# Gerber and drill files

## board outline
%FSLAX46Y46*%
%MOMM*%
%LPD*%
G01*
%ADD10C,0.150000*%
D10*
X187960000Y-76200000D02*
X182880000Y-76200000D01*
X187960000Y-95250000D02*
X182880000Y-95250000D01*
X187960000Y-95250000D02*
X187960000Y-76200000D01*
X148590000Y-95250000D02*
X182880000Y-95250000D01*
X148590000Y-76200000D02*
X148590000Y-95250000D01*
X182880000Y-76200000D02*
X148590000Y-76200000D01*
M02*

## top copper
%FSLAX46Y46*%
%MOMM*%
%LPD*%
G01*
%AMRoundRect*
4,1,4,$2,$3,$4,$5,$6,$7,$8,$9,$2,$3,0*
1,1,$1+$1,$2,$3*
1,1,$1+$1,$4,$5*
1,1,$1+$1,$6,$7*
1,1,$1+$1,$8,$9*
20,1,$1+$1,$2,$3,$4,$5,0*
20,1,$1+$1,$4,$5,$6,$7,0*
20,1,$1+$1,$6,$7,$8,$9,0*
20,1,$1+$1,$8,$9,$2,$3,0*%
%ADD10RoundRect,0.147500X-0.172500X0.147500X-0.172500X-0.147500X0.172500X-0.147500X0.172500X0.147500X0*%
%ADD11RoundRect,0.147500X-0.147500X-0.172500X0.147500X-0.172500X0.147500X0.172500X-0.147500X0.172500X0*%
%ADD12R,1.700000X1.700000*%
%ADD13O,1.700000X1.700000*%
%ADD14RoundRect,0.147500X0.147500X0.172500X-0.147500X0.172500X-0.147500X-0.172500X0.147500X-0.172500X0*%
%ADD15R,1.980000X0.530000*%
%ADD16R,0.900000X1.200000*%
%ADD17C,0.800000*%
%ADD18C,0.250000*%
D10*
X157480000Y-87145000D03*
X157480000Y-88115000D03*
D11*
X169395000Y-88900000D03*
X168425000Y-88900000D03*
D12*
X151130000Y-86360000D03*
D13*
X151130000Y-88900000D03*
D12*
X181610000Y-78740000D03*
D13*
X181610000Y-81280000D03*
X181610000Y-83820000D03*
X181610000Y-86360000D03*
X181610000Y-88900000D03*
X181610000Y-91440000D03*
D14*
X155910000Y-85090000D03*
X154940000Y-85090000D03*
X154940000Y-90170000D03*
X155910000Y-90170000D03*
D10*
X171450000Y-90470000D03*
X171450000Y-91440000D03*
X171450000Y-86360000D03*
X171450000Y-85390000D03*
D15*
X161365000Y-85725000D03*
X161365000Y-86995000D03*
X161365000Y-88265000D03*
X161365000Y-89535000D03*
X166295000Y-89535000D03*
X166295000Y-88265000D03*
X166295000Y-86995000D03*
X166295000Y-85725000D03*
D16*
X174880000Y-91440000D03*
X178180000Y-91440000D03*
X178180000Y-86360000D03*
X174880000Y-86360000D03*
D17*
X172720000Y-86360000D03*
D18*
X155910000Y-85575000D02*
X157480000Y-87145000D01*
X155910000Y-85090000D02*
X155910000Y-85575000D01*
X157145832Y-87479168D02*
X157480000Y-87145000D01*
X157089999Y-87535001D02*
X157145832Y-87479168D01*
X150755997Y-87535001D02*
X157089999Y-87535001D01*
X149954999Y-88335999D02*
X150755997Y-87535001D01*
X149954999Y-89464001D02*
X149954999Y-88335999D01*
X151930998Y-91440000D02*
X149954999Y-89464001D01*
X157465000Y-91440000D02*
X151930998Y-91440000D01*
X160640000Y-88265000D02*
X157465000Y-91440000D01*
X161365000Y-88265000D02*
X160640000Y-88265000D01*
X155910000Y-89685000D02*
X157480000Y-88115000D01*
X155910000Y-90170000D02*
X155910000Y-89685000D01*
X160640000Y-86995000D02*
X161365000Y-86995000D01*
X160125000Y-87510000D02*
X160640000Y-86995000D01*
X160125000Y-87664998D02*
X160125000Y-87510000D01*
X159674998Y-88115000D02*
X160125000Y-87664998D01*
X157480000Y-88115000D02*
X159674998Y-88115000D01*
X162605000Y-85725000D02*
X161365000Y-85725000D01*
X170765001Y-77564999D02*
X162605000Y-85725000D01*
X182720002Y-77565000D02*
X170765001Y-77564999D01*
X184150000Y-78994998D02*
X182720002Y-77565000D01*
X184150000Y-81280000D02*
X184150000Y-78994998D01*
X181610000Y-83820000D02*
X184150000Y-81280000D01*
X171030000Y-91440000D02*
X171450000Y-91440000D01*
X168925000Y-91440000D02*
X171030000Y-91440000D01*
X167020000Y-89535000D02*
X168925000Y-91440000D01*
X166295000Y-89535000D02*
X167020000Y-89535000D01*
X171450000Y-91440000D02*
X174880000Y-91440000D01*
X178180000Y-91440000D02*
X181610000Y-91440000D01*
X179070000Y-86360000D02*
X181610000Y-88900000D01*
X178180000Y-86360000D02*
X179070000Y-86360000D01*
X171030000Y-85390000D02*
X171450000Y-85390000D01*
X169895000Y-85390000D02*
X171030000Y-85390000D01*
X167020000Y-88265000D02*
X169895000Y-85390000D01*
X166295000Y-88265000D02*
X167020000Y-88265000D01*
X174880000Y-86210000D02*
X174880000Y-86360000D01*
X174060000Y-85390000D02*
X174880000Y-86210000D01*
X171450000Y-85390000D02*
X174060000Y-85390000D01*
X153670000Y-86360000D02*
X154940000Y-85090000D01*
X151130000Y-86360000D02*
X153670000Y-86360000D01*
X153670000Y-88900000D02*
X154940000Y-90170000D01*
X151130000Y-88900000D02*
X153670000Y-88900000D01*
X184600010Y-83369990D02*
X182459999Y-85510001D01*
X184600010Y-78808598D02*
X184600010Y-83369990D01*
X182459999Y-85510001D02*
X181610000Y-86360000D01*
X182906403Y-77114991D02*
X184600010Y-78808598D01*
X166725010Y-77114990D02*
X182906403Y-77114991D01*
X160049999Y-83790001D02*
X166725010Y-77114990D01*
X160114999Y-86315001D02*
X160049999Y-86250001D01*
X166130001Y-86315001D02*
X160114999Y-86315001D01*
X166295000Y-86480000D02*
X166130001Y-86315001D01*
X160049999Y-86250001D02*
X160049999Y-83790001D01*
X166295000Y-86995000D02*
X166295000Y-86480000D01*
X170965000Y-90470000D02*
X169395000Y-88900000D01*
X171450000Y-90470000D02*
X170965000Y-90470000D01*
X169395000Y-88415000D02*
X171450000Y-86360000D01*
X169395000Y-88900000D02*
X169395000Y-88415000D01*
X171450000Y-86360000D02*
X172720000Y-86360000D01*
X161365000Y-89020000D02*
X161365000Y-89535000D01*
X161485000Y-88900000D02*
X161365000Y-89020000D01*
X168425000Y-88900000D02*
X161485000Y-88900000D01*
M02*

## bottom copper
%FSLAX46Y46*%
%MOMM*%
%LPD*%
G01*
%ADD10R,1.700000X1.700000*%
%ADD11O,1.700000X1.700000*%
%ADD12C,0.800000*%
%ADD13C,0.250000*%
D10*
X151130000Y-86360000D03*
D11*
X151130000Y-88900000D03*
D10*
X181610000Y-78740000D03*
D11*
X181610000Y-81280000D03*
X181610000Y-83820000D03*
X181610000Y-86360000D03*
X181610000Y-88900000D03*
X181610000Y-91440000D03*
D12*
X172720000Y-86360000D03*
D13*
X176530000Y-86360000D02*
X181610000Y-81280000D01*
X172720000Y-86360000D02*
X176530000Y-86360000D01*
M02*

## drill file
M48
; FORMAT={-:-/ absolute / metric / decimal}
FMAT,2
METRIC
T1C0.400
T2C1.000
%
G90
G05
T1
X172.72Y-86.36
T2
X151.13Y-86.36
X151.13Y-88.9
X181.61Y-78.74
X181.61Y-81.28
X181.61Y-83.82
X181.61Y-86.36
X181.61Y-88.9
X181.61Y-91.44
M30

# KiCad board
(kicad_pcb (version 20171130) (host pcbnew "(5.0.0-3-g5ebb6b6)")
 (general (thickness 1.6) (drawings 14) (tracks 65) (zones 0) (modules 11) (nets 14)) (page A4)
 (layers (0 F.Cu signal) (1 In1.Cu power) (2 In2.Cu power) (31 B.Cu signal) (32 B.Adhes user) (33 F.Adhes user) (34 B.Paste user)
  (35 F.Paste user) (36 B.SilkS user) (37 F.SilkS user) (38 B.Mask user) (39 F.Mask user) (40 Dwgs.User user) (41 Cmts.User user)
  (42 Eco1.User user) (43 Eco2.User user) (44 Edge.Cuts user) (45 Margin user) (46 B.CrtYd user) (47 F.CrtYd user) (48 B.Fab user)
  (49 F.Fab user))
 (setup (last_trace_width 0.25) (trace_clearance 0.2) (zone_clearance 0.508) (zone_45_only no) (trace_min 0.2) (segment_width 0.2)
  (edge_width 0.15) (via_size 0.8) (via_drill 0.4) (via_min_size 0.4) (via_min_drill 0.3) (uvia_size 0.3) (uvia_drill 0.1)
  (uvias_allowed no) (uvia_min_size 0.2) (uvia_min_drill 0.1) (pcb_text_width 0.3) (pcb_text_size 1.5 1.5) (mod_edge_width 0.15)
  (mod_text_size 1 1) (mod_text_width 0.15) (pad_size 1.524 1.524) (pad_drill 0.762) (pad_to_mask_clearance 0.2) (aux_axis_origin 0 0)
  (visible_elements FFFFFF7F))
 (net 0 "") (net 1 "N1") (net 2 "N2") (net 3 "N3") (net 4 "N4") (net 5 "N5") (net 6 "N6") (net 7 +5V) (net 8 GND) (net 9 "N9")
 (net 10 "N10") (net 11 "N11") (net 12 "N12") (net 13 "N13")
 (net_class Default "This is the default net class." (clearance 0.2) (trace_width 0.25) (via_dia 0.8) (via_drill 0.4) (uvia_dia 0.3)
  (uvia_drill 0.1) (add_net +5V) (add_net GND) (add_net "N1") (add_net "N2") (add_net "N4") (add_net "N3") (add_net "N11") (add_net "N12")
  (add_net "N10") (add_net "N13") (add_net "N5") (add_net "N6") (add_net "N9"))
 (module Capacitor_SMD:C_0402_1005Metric (layer F.Cu) (at 157.48 87.63 270)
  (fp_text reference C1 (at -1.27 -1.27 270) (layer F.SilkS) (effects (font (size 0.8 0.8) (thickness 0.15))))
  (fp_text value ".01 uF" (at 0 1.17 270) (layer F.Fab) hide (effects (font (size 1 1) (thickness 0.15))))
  (pad 1 smd roundrect (at -0.485 0 270) (size 0.59 0.64) (layers F.Cu F.Paste F.Mask) (roundrect_rratio 0.25) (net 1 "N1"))
  (pad 2 smd roundrect (at 0.485 0 270) (size 0.59 0.64) (layers F.Cu F.Paste F.Mask) (roundrect_rratio 0.25) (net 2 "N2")))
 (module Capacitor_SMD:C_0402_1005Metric (layer F.Cu) (at 168.91 88.9)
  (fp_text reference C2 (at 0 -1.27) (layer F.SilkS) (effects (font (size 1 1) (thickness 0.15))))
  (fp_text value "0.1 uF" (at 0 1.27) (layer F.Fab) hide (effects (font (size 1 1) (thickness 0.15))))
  (pad 2 smd roundrect (at 0.485 0) (size 0.59 0.64) (layers F.Cu F.Paste F.Mask) (roundrect_rratio 0.25) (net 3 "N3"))
  (pad 1 smd roundrect (at -0.485 0) (size 0.59 0.64) (layers F.Cu F.Paste F.Mask) (roundrect_rratio 0.25) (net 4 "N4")))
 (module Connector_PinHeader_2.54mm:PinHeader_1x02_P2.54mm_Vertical (layer F.Cu) (at 151.13 86.36)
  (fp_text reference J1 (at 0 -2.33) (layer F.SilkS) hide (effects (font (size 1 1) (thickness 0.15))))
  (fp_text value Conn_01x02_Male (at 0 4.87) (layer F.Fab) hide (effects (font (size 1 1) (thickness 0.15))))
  (pad 1 thru_hole rect (at 0 0) (size 1.7 1.7) (drill 1) (layers *.Cu *.Mask) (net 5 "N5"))
  (pad 2 thru_hole oval (at 0 2.54) (size 1.7 1.7) (drill 1) (layers *.Cu *.Mask) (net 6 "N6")))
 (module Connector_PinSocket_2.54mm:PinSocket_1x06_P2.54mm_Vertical (layer F.Cu) (at 181.61 78.74)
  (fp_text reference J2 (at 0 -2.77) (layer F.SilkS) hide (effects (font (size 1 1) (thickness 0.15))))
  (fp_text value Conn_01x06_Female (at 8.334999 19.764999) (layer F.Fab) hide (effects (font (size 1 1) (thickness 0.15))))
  (pad 1 thru_hole rect (at 0 0) (size 1.7 1.7) (drill 1) (layers *.Cu *.Mask) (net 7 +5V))
  (pad 2 thru_hole oval (at 0 2.54) (size 1.7 1.7) (drill 1) (layers *.Cu *.Mask) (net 3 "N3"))
  (pad 3 thru_hole oval (at 0 5.08) (size 1.7 1.7) (drill 1) (layers *.Cu *.Mask) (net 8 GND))
  (pad 4 thru_hole oval (at 0 7.62) (size 1.7 1.7) (drill 1) (layers *.Cu *.Mask) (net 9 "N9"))
  (pad 5 thru_hole oval (at 0 10.16) (size 1.7 1.7) (drill 1) (layers *.Cu *.Mask) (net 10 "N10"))
  (pad 6 thru_hole oval (at 0 12.7) (size 1.7 1.7) (drill 1) (layers *.Cu *.Mask) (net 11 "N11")))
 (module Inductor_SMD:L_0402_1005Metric (layer F.Cu) (at 155.425 85.09 180)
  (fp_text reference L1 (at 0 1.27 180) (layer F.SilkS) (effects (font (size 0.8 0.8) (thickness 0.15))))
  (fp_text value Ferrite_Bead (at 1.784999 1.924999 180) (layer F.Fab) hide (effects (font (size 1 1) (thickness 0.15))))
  (pad 1 smd roundrect (at -0.485 0 180) (size 0.59 0.64) (layers F.Cu F.Paste F.Mask) (roundrect_rratio 0.25) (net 1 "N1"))
  (pad 2 smd roundrect (at 0.485 0 180) (size 0.59 0.64) (layers F.Cu F.Paste F.Mask) (roundrect_rratio 0.25) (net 5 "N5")))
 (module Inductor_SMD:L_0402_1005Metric (layer F.Cu) (at 155.425 90.17 180)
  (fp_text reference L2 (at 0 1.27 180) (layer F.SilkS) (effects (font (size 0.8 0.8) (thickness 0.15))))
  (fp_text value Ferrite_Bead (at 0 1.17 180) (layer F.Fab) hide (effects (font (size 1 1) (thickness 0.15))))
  (pad 2 smd roundrect (at 0.485 0 180) (size 0.59 0.64) (layers F.Cu F.Paste F.Mask) (roundrect_rratio 0.25) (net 6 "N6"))
  (pad 1 smd roundrect (at -0.485 0 180) (size 0.59 0.64) (layers F.Cu F.Paste F.Mask) (roundrect_rratio 0.25) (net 2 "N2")))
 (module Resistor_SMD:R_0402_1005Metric (layer F.Cu) (at 171.45 90.955 270)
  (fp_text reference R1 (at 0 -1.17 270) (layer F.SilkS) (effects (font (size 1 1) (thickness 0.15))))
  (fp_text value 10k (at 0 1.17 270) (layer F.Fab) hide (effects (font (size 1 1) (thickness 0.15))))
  (pad 1 smd roundrect (at -0.485 0 270) (size 0.59 0.64) (layers F.Cu F.Paste F.Mask) (roundrect_rratio 0.25) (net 3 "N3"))
  (pad 2 smd roundrect (at 0.485 0 270) (size 0.59 0.64) (layers F.Cu F.Paste F.Mask) (roundrect_rratio 0.25) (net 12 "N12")))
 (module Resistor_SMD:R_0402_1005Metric (layer F.Cu) (at 171.45 85.875 270)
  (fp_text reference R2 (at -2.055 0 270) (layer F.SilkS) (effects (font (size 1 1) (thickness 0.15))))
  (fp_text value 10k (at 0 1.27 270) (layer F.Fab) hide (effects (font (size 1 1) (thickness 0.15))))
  (pad 2 smd roundrect (at 0.485 0 270) (size 0.59 0.64) (layers F.Cu F.Paste F.Mask) (roundrect_rratio 0.25) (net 3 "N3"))
  (pad 1 smd roundrect (at -0.485 0 270) (size 0.59 0.64) (layers F.Cu F.Paste F.Mask) (roundrect_rratio 0.25) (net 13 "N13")))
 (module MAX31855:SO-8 (layer F.Cu) (at 163.83 87.63)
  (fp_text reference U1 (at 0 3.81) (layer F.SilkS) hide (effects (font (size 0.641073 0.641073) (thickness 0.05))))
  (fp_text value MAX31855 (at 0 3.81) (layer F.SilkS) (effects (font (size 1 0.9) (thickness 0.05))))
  (pad 1 smd rect (at -2.465 -1.905) (size 1.98 0.53) (layers F.Cu F.Paste F.Mask) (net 8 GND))
  (pad 2 smd rect (at -2.465 -0.635) (size 1.98 0.53) (layers F.Cu F.Paste F.Mask) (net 2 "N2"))
  (pad 3 smd rect (at -2.465 0.635) (size 1.98 0.53) (layers F.Cu F.Paste F.Mask) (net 1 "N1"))
  (pad 4 smd rect (at -2.465 1.905) (size 1.98 0.53) (layers F.Cu F.Paste F.Mask) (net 4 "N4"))
  (pad 5 smd rect (at 2.465 1.905) (size 1.98 0.53) (layers F.Cu F.Paste F.Mask) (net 12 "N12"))
  (pad 6 smd rect (at 2.465 0.635) (size 1.98 0.53) (layers F.Cu F.Paste F.Mask) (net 13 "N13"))
  (pad 7 smd rect (at 2.465 -0.635) (size 1.98 0.53) (layers F.Cu F.Paste F.Mask) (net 9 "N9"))
  (pad 8 smd rect (at 2.465 -1.905) (size 1.98 0.53) (layers F.Cu F.Paste F.Mask)))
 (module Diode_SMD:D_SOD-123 (layer F.Cu) (at 176.53 91.44 180)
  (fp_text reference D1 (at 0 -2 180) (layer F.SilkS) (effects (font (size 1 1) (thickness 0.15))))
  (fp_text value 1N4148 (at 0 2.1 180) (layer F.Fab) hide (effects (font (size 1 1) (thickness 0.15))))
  (pad 2 smd rect (at 1.65 0 180) (size 0.9 1.2) (layers F.Cu F.Paste F.Mask) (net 12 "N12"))
  (pad 1 smd rect (at -1.65 0 180) (size 0.9 1.2) (layers F.Cu F.Paste F.Mask) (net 11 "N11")))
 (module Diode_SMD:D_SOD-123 (layer F.Cu) (at 176.53 86.36 180)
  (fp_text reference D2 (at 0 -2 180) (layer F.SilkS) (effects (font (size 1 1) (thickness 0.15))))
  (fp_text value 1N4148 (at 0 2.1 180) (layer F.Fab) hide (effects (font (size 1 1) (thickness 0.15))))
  (pad 1 smd rect (at -1.65 0 180) (size 0.9 1.2) (layers F.Cu F.Paste F.Mask) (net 10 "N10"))
  (pad 2 smd rect (at 1.65 0 180) (size 0.9 1.2) (layers F.Cu F.Paste F.Mask) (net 13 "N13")))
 (gr_line (start 187.96 76.2) (end 182.88 76.2) (layer Edge.Cuts) (width 0.15))
 (gr_line (start 187.96 95.25) (end 182.88 95.25) (layer Edge.Cuts) (width 0.15))
 (gr_line (start 187.96 95.25) (end 187.96 76.2) (layer Edge.Cuts) (width 0.15))
 (gr_line (start 148.59 95.25) (end 182.88 95.25) (layer Edge.Cuts) (width 0.15))
 (gr_line (start 148.59 76.2) (end 148.59 95.25) (layer Edge.Cuts) (width 0.15))
 (gr_line (start 182.88 76.2) (end 148.59 76.2) (layer Edge.Cuts) (width 0.15))
 (segment (start 155.91 85.575) (end 157.48 87.145) (width 0.25) (layer F.Cu) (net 1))
 (segment (start 155.91 85.09) (end 155.91 85.575) (width 0.25) (layer F.Cu) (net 1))
 (segment (start 157.145832 87.479168) (end 157.48 87.145) (width 0.25) (layer F.Cu) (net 1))
 (segment (start 157.089999 87.535001) (end 157.145832 87.479168) (width 0.25) (layer F.Cu) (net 1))
 (segment (start 150.755997 87.535001) (end 157.089999 87.535001) (width 0.25) (layer F.Cu) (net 1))
 (segment (start 149.954999 88.335999) (end 150.755997 87.535001) (width 0.25) (layer F.Cu) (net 1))
 (segment (start 149.954999 89.464001) (end 149.954999 88.335999) (width 0.25) (layer F.Cu) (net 1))
 (segment (start 151.930998 91.44) (end 149.954999 89.464001) (width 0.25) (layer F.Cu) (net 1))
 (segment (start 157.465 91.44) (end 151.930998 91.44) (width 0.25) (layer F.Cu) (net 1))
 (segment (start 160.64 88.265) (end 157.465 91.44) (width 0.25) (layer F.Cu) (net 1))
 (segment (start 161.365 88.265) (end 160.64 88.265) (width 0.25) (layer F.Cu) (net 1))
 (segment (start 155.91 89.685) (end 157.48 88.115) (width 0.25) (layer F.Cu) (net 2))
 (segment (start 155.91 90.17) (end 155.91 89.685) (width 0.25) (layer F.Cu) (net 2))
 (segment (start 160.64 86.995) (end 161.365 86.995) (width 0.25) (layer F.Cu) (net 2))
 (segment (start 160.125 87.51) (end 160.64 86.995) (width 0.25) (layer F.Cu) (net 2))
 (segment (start 160.125 87.664998) (end 160.125 87.51) (width 0.25) (layer F.Cu) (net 2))
 (segment (start 159.674998 88.115) (end 160.125 87.664998) (width 0.25) (layer F.Cu) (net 2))
 (segment (start 157.48 88.115) (end 159.674998 88.115) (width 0.25) (layer F.Cu) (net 2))
 (segment (start 162.605 85.725) (end 161.365 85.725) (width 0.25) (layer F.Cu) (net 8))
 (segment (start 170.765001 77.564999) (end 162.605 85.725) (width 0.25) (layer F.Cu) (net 8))
 (segment (start 182.720002 77.565) (end 170.765001 77.564999) (width 0.25) (layer F.Cu) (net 8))
 (segment (start 184.15 78.994998) (end 182.720002 77.565) (width 0.25) (layer F.Cu) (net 8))
 (segment (start 184.15 81.28) (end 184.15 78.994998) (width 0.25) (layer F.Cu) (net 8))
 (segment (start 181.61 83.82) (end 184.15 81.28) (width 0.25) (layer F.Cu) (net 8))
 (segment (start 171.03 91.44) (end 171.45 91.44) (width 0.25) (layer F.Cu) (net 12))
 (segment (start 168.925 91.44) (end 171.03 91.44) (width 0.25) (layer F.Cu) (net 12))
 (segment (start 167.02 89.535) (end 168.925 91.44) (width 0.25) (layer F.Cu) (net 12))
 (segment (start 166.295 89.535) (end 167.02 89.535) (width 0.25) (layer F.Cu) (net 12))
 (segment (start 171.45 91.44) (end 174.88 91.44) (width 0.25) (layer F.Cu) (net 12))
 (segment (start 178.18 91.44) (end 181.61 91.44) (width 0.25) (layer F.Cu) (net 11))
 (segment (start 179.07 86.36) (end 181.61 88.9) (width 0.25) (layer F.Cu) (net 10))
 (segment (start 178.18 86.36) (end 179.07 86.36) (width 0.25) (layer F.Cu) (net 10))
 (segment (start 171.03 85.39) (end 171.45 85.39) (width 0.25) (layer F.Cu) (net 13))
 (segment (start 169.895 85.39) (end 171.03 85.39) (width 0.25) (layer F.Cu) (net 13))
 (segment (start 167.02 88.265) (end 169.895 85.39) (width 0.25) (layer F.Cu) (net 13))
 (segment (start 166.295 88.265) (end 167.02 88.265) (width 0.25) (layer F.Cu) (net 13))
 (segment (start 174.88 86.21) (end 174.88 86.36) (width 0.25) (layer F.Cu) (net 13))
 (segment (start 174.06 85.39) (end 174.88 86.21) (width 0.25) (layer F.Cu) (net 13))
 (segment (start 171.45 85.39) (end 174.06 85.39) (width 0.25) (layer F.Cu) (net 13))
 (segment (start 153.67 86.36) (end 154.94 85.09) (width 0.25) (layer F.Cu) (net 5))
 (segment (start 151.13 86.36) (end 153.67 86.36) (width 0.25) (layer F.Cu) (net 5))
 (segment (start 153.67 88.9) (end 154.94 90.17) (width 0.25) (layer F.Cu) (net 6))
 (segment (start 151.13 88.9) (end 153.67 88.9) (width 0.25) (layer F.Cu) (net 6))
 (segment (start 184.60001 83.36999) (end 182.459999 85.510001) (width 0.25) (layer F.Cu) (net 9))
 (segment (start 184.60001 78.808598) (end 184.60001 83.36999) (width 0.25) (layer F.Cu) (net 9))
 (segment (start 182.459999 85.510001) (end 181.61 86.36) (width 0.25) (layer F.Cu) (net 9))
 (segment (start 182.906403 77.114991) (end 184.60001 78.808598) (width 0.25) (layer F.Cu) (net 9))
 (segment (start 166.72501 77.11499) (end 182.906403 77.114991) (width 0.25) (layer F.Cu) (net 9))
 (segment (start 160.049999 83.790001) (end 166.72501 77.11499) (width 0.25) (layer F.Cu) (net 9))
 (segment (start 160.114999 86.315001) (end 160.049999 86.250001) (width 0.25) (layer F.Cu) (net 9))
 (segment (start 166.130001 86.315001) (end 160.114999 86.315001) (width 0.25) (layer F.Cu) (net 9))
 (segment (start 166.295 86.48) (end 166.130001 86.315001) (width 0.25) (layer F.Cu) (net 9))
 (segment (start 160.049999 86.250001) (end 160.049999 83.790001) (width 0.25) (layer F.Cu) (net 9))
 (segment (start 166.295 86.995) (end 166.295 86.48) (width 0.25) (layer F.Cu) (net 9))
 (segment (start 170.965 90.47) (end 169.395 88.9) (width 0.25) (layer F.Cu) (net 3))
 (segment (start 171.45 90.47) (end 170.965 90.47) (width 0.25) (layer F.Cu) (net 3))
 (segment (start 169.395 88.415) (end 171.45 86.36) (width 0.25) (layer F.Cu) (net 3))
 (segment (start 169.395 88.9) (end 169.395 88.415) (width 0.25) (layer F.Cu) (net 3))
 (via (at 172.72 86.36) (size 0.8) (drill 0.4) (layers F.Cu B.Cu) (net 3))
 (segment (start 171.45 86.36) (end 172.72 86.36) (width 0.25) (layer F.Cu) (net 3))
 (segment (start 176.53 86.36) (end 181.61 81.28) (width 0.25) (layer B.Cu) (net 3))
 (segment (start 172.72 86.36) (end 176.53 86.36) (width 0.25) (layer B.Cu) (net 3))
 (segment (start 161.365 89.02) (end 161.365 89.535) (width 0.25) (layer F.Cu) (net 4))
 (segment (start 161.485 88.9) (end 161.365 89.02) (width 0.25) (layer F.Cu) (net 4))
 (segment (start 168.425 88.9) (end 161.485 88.9) (width 0.25) (layer F.Cu) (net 4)))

